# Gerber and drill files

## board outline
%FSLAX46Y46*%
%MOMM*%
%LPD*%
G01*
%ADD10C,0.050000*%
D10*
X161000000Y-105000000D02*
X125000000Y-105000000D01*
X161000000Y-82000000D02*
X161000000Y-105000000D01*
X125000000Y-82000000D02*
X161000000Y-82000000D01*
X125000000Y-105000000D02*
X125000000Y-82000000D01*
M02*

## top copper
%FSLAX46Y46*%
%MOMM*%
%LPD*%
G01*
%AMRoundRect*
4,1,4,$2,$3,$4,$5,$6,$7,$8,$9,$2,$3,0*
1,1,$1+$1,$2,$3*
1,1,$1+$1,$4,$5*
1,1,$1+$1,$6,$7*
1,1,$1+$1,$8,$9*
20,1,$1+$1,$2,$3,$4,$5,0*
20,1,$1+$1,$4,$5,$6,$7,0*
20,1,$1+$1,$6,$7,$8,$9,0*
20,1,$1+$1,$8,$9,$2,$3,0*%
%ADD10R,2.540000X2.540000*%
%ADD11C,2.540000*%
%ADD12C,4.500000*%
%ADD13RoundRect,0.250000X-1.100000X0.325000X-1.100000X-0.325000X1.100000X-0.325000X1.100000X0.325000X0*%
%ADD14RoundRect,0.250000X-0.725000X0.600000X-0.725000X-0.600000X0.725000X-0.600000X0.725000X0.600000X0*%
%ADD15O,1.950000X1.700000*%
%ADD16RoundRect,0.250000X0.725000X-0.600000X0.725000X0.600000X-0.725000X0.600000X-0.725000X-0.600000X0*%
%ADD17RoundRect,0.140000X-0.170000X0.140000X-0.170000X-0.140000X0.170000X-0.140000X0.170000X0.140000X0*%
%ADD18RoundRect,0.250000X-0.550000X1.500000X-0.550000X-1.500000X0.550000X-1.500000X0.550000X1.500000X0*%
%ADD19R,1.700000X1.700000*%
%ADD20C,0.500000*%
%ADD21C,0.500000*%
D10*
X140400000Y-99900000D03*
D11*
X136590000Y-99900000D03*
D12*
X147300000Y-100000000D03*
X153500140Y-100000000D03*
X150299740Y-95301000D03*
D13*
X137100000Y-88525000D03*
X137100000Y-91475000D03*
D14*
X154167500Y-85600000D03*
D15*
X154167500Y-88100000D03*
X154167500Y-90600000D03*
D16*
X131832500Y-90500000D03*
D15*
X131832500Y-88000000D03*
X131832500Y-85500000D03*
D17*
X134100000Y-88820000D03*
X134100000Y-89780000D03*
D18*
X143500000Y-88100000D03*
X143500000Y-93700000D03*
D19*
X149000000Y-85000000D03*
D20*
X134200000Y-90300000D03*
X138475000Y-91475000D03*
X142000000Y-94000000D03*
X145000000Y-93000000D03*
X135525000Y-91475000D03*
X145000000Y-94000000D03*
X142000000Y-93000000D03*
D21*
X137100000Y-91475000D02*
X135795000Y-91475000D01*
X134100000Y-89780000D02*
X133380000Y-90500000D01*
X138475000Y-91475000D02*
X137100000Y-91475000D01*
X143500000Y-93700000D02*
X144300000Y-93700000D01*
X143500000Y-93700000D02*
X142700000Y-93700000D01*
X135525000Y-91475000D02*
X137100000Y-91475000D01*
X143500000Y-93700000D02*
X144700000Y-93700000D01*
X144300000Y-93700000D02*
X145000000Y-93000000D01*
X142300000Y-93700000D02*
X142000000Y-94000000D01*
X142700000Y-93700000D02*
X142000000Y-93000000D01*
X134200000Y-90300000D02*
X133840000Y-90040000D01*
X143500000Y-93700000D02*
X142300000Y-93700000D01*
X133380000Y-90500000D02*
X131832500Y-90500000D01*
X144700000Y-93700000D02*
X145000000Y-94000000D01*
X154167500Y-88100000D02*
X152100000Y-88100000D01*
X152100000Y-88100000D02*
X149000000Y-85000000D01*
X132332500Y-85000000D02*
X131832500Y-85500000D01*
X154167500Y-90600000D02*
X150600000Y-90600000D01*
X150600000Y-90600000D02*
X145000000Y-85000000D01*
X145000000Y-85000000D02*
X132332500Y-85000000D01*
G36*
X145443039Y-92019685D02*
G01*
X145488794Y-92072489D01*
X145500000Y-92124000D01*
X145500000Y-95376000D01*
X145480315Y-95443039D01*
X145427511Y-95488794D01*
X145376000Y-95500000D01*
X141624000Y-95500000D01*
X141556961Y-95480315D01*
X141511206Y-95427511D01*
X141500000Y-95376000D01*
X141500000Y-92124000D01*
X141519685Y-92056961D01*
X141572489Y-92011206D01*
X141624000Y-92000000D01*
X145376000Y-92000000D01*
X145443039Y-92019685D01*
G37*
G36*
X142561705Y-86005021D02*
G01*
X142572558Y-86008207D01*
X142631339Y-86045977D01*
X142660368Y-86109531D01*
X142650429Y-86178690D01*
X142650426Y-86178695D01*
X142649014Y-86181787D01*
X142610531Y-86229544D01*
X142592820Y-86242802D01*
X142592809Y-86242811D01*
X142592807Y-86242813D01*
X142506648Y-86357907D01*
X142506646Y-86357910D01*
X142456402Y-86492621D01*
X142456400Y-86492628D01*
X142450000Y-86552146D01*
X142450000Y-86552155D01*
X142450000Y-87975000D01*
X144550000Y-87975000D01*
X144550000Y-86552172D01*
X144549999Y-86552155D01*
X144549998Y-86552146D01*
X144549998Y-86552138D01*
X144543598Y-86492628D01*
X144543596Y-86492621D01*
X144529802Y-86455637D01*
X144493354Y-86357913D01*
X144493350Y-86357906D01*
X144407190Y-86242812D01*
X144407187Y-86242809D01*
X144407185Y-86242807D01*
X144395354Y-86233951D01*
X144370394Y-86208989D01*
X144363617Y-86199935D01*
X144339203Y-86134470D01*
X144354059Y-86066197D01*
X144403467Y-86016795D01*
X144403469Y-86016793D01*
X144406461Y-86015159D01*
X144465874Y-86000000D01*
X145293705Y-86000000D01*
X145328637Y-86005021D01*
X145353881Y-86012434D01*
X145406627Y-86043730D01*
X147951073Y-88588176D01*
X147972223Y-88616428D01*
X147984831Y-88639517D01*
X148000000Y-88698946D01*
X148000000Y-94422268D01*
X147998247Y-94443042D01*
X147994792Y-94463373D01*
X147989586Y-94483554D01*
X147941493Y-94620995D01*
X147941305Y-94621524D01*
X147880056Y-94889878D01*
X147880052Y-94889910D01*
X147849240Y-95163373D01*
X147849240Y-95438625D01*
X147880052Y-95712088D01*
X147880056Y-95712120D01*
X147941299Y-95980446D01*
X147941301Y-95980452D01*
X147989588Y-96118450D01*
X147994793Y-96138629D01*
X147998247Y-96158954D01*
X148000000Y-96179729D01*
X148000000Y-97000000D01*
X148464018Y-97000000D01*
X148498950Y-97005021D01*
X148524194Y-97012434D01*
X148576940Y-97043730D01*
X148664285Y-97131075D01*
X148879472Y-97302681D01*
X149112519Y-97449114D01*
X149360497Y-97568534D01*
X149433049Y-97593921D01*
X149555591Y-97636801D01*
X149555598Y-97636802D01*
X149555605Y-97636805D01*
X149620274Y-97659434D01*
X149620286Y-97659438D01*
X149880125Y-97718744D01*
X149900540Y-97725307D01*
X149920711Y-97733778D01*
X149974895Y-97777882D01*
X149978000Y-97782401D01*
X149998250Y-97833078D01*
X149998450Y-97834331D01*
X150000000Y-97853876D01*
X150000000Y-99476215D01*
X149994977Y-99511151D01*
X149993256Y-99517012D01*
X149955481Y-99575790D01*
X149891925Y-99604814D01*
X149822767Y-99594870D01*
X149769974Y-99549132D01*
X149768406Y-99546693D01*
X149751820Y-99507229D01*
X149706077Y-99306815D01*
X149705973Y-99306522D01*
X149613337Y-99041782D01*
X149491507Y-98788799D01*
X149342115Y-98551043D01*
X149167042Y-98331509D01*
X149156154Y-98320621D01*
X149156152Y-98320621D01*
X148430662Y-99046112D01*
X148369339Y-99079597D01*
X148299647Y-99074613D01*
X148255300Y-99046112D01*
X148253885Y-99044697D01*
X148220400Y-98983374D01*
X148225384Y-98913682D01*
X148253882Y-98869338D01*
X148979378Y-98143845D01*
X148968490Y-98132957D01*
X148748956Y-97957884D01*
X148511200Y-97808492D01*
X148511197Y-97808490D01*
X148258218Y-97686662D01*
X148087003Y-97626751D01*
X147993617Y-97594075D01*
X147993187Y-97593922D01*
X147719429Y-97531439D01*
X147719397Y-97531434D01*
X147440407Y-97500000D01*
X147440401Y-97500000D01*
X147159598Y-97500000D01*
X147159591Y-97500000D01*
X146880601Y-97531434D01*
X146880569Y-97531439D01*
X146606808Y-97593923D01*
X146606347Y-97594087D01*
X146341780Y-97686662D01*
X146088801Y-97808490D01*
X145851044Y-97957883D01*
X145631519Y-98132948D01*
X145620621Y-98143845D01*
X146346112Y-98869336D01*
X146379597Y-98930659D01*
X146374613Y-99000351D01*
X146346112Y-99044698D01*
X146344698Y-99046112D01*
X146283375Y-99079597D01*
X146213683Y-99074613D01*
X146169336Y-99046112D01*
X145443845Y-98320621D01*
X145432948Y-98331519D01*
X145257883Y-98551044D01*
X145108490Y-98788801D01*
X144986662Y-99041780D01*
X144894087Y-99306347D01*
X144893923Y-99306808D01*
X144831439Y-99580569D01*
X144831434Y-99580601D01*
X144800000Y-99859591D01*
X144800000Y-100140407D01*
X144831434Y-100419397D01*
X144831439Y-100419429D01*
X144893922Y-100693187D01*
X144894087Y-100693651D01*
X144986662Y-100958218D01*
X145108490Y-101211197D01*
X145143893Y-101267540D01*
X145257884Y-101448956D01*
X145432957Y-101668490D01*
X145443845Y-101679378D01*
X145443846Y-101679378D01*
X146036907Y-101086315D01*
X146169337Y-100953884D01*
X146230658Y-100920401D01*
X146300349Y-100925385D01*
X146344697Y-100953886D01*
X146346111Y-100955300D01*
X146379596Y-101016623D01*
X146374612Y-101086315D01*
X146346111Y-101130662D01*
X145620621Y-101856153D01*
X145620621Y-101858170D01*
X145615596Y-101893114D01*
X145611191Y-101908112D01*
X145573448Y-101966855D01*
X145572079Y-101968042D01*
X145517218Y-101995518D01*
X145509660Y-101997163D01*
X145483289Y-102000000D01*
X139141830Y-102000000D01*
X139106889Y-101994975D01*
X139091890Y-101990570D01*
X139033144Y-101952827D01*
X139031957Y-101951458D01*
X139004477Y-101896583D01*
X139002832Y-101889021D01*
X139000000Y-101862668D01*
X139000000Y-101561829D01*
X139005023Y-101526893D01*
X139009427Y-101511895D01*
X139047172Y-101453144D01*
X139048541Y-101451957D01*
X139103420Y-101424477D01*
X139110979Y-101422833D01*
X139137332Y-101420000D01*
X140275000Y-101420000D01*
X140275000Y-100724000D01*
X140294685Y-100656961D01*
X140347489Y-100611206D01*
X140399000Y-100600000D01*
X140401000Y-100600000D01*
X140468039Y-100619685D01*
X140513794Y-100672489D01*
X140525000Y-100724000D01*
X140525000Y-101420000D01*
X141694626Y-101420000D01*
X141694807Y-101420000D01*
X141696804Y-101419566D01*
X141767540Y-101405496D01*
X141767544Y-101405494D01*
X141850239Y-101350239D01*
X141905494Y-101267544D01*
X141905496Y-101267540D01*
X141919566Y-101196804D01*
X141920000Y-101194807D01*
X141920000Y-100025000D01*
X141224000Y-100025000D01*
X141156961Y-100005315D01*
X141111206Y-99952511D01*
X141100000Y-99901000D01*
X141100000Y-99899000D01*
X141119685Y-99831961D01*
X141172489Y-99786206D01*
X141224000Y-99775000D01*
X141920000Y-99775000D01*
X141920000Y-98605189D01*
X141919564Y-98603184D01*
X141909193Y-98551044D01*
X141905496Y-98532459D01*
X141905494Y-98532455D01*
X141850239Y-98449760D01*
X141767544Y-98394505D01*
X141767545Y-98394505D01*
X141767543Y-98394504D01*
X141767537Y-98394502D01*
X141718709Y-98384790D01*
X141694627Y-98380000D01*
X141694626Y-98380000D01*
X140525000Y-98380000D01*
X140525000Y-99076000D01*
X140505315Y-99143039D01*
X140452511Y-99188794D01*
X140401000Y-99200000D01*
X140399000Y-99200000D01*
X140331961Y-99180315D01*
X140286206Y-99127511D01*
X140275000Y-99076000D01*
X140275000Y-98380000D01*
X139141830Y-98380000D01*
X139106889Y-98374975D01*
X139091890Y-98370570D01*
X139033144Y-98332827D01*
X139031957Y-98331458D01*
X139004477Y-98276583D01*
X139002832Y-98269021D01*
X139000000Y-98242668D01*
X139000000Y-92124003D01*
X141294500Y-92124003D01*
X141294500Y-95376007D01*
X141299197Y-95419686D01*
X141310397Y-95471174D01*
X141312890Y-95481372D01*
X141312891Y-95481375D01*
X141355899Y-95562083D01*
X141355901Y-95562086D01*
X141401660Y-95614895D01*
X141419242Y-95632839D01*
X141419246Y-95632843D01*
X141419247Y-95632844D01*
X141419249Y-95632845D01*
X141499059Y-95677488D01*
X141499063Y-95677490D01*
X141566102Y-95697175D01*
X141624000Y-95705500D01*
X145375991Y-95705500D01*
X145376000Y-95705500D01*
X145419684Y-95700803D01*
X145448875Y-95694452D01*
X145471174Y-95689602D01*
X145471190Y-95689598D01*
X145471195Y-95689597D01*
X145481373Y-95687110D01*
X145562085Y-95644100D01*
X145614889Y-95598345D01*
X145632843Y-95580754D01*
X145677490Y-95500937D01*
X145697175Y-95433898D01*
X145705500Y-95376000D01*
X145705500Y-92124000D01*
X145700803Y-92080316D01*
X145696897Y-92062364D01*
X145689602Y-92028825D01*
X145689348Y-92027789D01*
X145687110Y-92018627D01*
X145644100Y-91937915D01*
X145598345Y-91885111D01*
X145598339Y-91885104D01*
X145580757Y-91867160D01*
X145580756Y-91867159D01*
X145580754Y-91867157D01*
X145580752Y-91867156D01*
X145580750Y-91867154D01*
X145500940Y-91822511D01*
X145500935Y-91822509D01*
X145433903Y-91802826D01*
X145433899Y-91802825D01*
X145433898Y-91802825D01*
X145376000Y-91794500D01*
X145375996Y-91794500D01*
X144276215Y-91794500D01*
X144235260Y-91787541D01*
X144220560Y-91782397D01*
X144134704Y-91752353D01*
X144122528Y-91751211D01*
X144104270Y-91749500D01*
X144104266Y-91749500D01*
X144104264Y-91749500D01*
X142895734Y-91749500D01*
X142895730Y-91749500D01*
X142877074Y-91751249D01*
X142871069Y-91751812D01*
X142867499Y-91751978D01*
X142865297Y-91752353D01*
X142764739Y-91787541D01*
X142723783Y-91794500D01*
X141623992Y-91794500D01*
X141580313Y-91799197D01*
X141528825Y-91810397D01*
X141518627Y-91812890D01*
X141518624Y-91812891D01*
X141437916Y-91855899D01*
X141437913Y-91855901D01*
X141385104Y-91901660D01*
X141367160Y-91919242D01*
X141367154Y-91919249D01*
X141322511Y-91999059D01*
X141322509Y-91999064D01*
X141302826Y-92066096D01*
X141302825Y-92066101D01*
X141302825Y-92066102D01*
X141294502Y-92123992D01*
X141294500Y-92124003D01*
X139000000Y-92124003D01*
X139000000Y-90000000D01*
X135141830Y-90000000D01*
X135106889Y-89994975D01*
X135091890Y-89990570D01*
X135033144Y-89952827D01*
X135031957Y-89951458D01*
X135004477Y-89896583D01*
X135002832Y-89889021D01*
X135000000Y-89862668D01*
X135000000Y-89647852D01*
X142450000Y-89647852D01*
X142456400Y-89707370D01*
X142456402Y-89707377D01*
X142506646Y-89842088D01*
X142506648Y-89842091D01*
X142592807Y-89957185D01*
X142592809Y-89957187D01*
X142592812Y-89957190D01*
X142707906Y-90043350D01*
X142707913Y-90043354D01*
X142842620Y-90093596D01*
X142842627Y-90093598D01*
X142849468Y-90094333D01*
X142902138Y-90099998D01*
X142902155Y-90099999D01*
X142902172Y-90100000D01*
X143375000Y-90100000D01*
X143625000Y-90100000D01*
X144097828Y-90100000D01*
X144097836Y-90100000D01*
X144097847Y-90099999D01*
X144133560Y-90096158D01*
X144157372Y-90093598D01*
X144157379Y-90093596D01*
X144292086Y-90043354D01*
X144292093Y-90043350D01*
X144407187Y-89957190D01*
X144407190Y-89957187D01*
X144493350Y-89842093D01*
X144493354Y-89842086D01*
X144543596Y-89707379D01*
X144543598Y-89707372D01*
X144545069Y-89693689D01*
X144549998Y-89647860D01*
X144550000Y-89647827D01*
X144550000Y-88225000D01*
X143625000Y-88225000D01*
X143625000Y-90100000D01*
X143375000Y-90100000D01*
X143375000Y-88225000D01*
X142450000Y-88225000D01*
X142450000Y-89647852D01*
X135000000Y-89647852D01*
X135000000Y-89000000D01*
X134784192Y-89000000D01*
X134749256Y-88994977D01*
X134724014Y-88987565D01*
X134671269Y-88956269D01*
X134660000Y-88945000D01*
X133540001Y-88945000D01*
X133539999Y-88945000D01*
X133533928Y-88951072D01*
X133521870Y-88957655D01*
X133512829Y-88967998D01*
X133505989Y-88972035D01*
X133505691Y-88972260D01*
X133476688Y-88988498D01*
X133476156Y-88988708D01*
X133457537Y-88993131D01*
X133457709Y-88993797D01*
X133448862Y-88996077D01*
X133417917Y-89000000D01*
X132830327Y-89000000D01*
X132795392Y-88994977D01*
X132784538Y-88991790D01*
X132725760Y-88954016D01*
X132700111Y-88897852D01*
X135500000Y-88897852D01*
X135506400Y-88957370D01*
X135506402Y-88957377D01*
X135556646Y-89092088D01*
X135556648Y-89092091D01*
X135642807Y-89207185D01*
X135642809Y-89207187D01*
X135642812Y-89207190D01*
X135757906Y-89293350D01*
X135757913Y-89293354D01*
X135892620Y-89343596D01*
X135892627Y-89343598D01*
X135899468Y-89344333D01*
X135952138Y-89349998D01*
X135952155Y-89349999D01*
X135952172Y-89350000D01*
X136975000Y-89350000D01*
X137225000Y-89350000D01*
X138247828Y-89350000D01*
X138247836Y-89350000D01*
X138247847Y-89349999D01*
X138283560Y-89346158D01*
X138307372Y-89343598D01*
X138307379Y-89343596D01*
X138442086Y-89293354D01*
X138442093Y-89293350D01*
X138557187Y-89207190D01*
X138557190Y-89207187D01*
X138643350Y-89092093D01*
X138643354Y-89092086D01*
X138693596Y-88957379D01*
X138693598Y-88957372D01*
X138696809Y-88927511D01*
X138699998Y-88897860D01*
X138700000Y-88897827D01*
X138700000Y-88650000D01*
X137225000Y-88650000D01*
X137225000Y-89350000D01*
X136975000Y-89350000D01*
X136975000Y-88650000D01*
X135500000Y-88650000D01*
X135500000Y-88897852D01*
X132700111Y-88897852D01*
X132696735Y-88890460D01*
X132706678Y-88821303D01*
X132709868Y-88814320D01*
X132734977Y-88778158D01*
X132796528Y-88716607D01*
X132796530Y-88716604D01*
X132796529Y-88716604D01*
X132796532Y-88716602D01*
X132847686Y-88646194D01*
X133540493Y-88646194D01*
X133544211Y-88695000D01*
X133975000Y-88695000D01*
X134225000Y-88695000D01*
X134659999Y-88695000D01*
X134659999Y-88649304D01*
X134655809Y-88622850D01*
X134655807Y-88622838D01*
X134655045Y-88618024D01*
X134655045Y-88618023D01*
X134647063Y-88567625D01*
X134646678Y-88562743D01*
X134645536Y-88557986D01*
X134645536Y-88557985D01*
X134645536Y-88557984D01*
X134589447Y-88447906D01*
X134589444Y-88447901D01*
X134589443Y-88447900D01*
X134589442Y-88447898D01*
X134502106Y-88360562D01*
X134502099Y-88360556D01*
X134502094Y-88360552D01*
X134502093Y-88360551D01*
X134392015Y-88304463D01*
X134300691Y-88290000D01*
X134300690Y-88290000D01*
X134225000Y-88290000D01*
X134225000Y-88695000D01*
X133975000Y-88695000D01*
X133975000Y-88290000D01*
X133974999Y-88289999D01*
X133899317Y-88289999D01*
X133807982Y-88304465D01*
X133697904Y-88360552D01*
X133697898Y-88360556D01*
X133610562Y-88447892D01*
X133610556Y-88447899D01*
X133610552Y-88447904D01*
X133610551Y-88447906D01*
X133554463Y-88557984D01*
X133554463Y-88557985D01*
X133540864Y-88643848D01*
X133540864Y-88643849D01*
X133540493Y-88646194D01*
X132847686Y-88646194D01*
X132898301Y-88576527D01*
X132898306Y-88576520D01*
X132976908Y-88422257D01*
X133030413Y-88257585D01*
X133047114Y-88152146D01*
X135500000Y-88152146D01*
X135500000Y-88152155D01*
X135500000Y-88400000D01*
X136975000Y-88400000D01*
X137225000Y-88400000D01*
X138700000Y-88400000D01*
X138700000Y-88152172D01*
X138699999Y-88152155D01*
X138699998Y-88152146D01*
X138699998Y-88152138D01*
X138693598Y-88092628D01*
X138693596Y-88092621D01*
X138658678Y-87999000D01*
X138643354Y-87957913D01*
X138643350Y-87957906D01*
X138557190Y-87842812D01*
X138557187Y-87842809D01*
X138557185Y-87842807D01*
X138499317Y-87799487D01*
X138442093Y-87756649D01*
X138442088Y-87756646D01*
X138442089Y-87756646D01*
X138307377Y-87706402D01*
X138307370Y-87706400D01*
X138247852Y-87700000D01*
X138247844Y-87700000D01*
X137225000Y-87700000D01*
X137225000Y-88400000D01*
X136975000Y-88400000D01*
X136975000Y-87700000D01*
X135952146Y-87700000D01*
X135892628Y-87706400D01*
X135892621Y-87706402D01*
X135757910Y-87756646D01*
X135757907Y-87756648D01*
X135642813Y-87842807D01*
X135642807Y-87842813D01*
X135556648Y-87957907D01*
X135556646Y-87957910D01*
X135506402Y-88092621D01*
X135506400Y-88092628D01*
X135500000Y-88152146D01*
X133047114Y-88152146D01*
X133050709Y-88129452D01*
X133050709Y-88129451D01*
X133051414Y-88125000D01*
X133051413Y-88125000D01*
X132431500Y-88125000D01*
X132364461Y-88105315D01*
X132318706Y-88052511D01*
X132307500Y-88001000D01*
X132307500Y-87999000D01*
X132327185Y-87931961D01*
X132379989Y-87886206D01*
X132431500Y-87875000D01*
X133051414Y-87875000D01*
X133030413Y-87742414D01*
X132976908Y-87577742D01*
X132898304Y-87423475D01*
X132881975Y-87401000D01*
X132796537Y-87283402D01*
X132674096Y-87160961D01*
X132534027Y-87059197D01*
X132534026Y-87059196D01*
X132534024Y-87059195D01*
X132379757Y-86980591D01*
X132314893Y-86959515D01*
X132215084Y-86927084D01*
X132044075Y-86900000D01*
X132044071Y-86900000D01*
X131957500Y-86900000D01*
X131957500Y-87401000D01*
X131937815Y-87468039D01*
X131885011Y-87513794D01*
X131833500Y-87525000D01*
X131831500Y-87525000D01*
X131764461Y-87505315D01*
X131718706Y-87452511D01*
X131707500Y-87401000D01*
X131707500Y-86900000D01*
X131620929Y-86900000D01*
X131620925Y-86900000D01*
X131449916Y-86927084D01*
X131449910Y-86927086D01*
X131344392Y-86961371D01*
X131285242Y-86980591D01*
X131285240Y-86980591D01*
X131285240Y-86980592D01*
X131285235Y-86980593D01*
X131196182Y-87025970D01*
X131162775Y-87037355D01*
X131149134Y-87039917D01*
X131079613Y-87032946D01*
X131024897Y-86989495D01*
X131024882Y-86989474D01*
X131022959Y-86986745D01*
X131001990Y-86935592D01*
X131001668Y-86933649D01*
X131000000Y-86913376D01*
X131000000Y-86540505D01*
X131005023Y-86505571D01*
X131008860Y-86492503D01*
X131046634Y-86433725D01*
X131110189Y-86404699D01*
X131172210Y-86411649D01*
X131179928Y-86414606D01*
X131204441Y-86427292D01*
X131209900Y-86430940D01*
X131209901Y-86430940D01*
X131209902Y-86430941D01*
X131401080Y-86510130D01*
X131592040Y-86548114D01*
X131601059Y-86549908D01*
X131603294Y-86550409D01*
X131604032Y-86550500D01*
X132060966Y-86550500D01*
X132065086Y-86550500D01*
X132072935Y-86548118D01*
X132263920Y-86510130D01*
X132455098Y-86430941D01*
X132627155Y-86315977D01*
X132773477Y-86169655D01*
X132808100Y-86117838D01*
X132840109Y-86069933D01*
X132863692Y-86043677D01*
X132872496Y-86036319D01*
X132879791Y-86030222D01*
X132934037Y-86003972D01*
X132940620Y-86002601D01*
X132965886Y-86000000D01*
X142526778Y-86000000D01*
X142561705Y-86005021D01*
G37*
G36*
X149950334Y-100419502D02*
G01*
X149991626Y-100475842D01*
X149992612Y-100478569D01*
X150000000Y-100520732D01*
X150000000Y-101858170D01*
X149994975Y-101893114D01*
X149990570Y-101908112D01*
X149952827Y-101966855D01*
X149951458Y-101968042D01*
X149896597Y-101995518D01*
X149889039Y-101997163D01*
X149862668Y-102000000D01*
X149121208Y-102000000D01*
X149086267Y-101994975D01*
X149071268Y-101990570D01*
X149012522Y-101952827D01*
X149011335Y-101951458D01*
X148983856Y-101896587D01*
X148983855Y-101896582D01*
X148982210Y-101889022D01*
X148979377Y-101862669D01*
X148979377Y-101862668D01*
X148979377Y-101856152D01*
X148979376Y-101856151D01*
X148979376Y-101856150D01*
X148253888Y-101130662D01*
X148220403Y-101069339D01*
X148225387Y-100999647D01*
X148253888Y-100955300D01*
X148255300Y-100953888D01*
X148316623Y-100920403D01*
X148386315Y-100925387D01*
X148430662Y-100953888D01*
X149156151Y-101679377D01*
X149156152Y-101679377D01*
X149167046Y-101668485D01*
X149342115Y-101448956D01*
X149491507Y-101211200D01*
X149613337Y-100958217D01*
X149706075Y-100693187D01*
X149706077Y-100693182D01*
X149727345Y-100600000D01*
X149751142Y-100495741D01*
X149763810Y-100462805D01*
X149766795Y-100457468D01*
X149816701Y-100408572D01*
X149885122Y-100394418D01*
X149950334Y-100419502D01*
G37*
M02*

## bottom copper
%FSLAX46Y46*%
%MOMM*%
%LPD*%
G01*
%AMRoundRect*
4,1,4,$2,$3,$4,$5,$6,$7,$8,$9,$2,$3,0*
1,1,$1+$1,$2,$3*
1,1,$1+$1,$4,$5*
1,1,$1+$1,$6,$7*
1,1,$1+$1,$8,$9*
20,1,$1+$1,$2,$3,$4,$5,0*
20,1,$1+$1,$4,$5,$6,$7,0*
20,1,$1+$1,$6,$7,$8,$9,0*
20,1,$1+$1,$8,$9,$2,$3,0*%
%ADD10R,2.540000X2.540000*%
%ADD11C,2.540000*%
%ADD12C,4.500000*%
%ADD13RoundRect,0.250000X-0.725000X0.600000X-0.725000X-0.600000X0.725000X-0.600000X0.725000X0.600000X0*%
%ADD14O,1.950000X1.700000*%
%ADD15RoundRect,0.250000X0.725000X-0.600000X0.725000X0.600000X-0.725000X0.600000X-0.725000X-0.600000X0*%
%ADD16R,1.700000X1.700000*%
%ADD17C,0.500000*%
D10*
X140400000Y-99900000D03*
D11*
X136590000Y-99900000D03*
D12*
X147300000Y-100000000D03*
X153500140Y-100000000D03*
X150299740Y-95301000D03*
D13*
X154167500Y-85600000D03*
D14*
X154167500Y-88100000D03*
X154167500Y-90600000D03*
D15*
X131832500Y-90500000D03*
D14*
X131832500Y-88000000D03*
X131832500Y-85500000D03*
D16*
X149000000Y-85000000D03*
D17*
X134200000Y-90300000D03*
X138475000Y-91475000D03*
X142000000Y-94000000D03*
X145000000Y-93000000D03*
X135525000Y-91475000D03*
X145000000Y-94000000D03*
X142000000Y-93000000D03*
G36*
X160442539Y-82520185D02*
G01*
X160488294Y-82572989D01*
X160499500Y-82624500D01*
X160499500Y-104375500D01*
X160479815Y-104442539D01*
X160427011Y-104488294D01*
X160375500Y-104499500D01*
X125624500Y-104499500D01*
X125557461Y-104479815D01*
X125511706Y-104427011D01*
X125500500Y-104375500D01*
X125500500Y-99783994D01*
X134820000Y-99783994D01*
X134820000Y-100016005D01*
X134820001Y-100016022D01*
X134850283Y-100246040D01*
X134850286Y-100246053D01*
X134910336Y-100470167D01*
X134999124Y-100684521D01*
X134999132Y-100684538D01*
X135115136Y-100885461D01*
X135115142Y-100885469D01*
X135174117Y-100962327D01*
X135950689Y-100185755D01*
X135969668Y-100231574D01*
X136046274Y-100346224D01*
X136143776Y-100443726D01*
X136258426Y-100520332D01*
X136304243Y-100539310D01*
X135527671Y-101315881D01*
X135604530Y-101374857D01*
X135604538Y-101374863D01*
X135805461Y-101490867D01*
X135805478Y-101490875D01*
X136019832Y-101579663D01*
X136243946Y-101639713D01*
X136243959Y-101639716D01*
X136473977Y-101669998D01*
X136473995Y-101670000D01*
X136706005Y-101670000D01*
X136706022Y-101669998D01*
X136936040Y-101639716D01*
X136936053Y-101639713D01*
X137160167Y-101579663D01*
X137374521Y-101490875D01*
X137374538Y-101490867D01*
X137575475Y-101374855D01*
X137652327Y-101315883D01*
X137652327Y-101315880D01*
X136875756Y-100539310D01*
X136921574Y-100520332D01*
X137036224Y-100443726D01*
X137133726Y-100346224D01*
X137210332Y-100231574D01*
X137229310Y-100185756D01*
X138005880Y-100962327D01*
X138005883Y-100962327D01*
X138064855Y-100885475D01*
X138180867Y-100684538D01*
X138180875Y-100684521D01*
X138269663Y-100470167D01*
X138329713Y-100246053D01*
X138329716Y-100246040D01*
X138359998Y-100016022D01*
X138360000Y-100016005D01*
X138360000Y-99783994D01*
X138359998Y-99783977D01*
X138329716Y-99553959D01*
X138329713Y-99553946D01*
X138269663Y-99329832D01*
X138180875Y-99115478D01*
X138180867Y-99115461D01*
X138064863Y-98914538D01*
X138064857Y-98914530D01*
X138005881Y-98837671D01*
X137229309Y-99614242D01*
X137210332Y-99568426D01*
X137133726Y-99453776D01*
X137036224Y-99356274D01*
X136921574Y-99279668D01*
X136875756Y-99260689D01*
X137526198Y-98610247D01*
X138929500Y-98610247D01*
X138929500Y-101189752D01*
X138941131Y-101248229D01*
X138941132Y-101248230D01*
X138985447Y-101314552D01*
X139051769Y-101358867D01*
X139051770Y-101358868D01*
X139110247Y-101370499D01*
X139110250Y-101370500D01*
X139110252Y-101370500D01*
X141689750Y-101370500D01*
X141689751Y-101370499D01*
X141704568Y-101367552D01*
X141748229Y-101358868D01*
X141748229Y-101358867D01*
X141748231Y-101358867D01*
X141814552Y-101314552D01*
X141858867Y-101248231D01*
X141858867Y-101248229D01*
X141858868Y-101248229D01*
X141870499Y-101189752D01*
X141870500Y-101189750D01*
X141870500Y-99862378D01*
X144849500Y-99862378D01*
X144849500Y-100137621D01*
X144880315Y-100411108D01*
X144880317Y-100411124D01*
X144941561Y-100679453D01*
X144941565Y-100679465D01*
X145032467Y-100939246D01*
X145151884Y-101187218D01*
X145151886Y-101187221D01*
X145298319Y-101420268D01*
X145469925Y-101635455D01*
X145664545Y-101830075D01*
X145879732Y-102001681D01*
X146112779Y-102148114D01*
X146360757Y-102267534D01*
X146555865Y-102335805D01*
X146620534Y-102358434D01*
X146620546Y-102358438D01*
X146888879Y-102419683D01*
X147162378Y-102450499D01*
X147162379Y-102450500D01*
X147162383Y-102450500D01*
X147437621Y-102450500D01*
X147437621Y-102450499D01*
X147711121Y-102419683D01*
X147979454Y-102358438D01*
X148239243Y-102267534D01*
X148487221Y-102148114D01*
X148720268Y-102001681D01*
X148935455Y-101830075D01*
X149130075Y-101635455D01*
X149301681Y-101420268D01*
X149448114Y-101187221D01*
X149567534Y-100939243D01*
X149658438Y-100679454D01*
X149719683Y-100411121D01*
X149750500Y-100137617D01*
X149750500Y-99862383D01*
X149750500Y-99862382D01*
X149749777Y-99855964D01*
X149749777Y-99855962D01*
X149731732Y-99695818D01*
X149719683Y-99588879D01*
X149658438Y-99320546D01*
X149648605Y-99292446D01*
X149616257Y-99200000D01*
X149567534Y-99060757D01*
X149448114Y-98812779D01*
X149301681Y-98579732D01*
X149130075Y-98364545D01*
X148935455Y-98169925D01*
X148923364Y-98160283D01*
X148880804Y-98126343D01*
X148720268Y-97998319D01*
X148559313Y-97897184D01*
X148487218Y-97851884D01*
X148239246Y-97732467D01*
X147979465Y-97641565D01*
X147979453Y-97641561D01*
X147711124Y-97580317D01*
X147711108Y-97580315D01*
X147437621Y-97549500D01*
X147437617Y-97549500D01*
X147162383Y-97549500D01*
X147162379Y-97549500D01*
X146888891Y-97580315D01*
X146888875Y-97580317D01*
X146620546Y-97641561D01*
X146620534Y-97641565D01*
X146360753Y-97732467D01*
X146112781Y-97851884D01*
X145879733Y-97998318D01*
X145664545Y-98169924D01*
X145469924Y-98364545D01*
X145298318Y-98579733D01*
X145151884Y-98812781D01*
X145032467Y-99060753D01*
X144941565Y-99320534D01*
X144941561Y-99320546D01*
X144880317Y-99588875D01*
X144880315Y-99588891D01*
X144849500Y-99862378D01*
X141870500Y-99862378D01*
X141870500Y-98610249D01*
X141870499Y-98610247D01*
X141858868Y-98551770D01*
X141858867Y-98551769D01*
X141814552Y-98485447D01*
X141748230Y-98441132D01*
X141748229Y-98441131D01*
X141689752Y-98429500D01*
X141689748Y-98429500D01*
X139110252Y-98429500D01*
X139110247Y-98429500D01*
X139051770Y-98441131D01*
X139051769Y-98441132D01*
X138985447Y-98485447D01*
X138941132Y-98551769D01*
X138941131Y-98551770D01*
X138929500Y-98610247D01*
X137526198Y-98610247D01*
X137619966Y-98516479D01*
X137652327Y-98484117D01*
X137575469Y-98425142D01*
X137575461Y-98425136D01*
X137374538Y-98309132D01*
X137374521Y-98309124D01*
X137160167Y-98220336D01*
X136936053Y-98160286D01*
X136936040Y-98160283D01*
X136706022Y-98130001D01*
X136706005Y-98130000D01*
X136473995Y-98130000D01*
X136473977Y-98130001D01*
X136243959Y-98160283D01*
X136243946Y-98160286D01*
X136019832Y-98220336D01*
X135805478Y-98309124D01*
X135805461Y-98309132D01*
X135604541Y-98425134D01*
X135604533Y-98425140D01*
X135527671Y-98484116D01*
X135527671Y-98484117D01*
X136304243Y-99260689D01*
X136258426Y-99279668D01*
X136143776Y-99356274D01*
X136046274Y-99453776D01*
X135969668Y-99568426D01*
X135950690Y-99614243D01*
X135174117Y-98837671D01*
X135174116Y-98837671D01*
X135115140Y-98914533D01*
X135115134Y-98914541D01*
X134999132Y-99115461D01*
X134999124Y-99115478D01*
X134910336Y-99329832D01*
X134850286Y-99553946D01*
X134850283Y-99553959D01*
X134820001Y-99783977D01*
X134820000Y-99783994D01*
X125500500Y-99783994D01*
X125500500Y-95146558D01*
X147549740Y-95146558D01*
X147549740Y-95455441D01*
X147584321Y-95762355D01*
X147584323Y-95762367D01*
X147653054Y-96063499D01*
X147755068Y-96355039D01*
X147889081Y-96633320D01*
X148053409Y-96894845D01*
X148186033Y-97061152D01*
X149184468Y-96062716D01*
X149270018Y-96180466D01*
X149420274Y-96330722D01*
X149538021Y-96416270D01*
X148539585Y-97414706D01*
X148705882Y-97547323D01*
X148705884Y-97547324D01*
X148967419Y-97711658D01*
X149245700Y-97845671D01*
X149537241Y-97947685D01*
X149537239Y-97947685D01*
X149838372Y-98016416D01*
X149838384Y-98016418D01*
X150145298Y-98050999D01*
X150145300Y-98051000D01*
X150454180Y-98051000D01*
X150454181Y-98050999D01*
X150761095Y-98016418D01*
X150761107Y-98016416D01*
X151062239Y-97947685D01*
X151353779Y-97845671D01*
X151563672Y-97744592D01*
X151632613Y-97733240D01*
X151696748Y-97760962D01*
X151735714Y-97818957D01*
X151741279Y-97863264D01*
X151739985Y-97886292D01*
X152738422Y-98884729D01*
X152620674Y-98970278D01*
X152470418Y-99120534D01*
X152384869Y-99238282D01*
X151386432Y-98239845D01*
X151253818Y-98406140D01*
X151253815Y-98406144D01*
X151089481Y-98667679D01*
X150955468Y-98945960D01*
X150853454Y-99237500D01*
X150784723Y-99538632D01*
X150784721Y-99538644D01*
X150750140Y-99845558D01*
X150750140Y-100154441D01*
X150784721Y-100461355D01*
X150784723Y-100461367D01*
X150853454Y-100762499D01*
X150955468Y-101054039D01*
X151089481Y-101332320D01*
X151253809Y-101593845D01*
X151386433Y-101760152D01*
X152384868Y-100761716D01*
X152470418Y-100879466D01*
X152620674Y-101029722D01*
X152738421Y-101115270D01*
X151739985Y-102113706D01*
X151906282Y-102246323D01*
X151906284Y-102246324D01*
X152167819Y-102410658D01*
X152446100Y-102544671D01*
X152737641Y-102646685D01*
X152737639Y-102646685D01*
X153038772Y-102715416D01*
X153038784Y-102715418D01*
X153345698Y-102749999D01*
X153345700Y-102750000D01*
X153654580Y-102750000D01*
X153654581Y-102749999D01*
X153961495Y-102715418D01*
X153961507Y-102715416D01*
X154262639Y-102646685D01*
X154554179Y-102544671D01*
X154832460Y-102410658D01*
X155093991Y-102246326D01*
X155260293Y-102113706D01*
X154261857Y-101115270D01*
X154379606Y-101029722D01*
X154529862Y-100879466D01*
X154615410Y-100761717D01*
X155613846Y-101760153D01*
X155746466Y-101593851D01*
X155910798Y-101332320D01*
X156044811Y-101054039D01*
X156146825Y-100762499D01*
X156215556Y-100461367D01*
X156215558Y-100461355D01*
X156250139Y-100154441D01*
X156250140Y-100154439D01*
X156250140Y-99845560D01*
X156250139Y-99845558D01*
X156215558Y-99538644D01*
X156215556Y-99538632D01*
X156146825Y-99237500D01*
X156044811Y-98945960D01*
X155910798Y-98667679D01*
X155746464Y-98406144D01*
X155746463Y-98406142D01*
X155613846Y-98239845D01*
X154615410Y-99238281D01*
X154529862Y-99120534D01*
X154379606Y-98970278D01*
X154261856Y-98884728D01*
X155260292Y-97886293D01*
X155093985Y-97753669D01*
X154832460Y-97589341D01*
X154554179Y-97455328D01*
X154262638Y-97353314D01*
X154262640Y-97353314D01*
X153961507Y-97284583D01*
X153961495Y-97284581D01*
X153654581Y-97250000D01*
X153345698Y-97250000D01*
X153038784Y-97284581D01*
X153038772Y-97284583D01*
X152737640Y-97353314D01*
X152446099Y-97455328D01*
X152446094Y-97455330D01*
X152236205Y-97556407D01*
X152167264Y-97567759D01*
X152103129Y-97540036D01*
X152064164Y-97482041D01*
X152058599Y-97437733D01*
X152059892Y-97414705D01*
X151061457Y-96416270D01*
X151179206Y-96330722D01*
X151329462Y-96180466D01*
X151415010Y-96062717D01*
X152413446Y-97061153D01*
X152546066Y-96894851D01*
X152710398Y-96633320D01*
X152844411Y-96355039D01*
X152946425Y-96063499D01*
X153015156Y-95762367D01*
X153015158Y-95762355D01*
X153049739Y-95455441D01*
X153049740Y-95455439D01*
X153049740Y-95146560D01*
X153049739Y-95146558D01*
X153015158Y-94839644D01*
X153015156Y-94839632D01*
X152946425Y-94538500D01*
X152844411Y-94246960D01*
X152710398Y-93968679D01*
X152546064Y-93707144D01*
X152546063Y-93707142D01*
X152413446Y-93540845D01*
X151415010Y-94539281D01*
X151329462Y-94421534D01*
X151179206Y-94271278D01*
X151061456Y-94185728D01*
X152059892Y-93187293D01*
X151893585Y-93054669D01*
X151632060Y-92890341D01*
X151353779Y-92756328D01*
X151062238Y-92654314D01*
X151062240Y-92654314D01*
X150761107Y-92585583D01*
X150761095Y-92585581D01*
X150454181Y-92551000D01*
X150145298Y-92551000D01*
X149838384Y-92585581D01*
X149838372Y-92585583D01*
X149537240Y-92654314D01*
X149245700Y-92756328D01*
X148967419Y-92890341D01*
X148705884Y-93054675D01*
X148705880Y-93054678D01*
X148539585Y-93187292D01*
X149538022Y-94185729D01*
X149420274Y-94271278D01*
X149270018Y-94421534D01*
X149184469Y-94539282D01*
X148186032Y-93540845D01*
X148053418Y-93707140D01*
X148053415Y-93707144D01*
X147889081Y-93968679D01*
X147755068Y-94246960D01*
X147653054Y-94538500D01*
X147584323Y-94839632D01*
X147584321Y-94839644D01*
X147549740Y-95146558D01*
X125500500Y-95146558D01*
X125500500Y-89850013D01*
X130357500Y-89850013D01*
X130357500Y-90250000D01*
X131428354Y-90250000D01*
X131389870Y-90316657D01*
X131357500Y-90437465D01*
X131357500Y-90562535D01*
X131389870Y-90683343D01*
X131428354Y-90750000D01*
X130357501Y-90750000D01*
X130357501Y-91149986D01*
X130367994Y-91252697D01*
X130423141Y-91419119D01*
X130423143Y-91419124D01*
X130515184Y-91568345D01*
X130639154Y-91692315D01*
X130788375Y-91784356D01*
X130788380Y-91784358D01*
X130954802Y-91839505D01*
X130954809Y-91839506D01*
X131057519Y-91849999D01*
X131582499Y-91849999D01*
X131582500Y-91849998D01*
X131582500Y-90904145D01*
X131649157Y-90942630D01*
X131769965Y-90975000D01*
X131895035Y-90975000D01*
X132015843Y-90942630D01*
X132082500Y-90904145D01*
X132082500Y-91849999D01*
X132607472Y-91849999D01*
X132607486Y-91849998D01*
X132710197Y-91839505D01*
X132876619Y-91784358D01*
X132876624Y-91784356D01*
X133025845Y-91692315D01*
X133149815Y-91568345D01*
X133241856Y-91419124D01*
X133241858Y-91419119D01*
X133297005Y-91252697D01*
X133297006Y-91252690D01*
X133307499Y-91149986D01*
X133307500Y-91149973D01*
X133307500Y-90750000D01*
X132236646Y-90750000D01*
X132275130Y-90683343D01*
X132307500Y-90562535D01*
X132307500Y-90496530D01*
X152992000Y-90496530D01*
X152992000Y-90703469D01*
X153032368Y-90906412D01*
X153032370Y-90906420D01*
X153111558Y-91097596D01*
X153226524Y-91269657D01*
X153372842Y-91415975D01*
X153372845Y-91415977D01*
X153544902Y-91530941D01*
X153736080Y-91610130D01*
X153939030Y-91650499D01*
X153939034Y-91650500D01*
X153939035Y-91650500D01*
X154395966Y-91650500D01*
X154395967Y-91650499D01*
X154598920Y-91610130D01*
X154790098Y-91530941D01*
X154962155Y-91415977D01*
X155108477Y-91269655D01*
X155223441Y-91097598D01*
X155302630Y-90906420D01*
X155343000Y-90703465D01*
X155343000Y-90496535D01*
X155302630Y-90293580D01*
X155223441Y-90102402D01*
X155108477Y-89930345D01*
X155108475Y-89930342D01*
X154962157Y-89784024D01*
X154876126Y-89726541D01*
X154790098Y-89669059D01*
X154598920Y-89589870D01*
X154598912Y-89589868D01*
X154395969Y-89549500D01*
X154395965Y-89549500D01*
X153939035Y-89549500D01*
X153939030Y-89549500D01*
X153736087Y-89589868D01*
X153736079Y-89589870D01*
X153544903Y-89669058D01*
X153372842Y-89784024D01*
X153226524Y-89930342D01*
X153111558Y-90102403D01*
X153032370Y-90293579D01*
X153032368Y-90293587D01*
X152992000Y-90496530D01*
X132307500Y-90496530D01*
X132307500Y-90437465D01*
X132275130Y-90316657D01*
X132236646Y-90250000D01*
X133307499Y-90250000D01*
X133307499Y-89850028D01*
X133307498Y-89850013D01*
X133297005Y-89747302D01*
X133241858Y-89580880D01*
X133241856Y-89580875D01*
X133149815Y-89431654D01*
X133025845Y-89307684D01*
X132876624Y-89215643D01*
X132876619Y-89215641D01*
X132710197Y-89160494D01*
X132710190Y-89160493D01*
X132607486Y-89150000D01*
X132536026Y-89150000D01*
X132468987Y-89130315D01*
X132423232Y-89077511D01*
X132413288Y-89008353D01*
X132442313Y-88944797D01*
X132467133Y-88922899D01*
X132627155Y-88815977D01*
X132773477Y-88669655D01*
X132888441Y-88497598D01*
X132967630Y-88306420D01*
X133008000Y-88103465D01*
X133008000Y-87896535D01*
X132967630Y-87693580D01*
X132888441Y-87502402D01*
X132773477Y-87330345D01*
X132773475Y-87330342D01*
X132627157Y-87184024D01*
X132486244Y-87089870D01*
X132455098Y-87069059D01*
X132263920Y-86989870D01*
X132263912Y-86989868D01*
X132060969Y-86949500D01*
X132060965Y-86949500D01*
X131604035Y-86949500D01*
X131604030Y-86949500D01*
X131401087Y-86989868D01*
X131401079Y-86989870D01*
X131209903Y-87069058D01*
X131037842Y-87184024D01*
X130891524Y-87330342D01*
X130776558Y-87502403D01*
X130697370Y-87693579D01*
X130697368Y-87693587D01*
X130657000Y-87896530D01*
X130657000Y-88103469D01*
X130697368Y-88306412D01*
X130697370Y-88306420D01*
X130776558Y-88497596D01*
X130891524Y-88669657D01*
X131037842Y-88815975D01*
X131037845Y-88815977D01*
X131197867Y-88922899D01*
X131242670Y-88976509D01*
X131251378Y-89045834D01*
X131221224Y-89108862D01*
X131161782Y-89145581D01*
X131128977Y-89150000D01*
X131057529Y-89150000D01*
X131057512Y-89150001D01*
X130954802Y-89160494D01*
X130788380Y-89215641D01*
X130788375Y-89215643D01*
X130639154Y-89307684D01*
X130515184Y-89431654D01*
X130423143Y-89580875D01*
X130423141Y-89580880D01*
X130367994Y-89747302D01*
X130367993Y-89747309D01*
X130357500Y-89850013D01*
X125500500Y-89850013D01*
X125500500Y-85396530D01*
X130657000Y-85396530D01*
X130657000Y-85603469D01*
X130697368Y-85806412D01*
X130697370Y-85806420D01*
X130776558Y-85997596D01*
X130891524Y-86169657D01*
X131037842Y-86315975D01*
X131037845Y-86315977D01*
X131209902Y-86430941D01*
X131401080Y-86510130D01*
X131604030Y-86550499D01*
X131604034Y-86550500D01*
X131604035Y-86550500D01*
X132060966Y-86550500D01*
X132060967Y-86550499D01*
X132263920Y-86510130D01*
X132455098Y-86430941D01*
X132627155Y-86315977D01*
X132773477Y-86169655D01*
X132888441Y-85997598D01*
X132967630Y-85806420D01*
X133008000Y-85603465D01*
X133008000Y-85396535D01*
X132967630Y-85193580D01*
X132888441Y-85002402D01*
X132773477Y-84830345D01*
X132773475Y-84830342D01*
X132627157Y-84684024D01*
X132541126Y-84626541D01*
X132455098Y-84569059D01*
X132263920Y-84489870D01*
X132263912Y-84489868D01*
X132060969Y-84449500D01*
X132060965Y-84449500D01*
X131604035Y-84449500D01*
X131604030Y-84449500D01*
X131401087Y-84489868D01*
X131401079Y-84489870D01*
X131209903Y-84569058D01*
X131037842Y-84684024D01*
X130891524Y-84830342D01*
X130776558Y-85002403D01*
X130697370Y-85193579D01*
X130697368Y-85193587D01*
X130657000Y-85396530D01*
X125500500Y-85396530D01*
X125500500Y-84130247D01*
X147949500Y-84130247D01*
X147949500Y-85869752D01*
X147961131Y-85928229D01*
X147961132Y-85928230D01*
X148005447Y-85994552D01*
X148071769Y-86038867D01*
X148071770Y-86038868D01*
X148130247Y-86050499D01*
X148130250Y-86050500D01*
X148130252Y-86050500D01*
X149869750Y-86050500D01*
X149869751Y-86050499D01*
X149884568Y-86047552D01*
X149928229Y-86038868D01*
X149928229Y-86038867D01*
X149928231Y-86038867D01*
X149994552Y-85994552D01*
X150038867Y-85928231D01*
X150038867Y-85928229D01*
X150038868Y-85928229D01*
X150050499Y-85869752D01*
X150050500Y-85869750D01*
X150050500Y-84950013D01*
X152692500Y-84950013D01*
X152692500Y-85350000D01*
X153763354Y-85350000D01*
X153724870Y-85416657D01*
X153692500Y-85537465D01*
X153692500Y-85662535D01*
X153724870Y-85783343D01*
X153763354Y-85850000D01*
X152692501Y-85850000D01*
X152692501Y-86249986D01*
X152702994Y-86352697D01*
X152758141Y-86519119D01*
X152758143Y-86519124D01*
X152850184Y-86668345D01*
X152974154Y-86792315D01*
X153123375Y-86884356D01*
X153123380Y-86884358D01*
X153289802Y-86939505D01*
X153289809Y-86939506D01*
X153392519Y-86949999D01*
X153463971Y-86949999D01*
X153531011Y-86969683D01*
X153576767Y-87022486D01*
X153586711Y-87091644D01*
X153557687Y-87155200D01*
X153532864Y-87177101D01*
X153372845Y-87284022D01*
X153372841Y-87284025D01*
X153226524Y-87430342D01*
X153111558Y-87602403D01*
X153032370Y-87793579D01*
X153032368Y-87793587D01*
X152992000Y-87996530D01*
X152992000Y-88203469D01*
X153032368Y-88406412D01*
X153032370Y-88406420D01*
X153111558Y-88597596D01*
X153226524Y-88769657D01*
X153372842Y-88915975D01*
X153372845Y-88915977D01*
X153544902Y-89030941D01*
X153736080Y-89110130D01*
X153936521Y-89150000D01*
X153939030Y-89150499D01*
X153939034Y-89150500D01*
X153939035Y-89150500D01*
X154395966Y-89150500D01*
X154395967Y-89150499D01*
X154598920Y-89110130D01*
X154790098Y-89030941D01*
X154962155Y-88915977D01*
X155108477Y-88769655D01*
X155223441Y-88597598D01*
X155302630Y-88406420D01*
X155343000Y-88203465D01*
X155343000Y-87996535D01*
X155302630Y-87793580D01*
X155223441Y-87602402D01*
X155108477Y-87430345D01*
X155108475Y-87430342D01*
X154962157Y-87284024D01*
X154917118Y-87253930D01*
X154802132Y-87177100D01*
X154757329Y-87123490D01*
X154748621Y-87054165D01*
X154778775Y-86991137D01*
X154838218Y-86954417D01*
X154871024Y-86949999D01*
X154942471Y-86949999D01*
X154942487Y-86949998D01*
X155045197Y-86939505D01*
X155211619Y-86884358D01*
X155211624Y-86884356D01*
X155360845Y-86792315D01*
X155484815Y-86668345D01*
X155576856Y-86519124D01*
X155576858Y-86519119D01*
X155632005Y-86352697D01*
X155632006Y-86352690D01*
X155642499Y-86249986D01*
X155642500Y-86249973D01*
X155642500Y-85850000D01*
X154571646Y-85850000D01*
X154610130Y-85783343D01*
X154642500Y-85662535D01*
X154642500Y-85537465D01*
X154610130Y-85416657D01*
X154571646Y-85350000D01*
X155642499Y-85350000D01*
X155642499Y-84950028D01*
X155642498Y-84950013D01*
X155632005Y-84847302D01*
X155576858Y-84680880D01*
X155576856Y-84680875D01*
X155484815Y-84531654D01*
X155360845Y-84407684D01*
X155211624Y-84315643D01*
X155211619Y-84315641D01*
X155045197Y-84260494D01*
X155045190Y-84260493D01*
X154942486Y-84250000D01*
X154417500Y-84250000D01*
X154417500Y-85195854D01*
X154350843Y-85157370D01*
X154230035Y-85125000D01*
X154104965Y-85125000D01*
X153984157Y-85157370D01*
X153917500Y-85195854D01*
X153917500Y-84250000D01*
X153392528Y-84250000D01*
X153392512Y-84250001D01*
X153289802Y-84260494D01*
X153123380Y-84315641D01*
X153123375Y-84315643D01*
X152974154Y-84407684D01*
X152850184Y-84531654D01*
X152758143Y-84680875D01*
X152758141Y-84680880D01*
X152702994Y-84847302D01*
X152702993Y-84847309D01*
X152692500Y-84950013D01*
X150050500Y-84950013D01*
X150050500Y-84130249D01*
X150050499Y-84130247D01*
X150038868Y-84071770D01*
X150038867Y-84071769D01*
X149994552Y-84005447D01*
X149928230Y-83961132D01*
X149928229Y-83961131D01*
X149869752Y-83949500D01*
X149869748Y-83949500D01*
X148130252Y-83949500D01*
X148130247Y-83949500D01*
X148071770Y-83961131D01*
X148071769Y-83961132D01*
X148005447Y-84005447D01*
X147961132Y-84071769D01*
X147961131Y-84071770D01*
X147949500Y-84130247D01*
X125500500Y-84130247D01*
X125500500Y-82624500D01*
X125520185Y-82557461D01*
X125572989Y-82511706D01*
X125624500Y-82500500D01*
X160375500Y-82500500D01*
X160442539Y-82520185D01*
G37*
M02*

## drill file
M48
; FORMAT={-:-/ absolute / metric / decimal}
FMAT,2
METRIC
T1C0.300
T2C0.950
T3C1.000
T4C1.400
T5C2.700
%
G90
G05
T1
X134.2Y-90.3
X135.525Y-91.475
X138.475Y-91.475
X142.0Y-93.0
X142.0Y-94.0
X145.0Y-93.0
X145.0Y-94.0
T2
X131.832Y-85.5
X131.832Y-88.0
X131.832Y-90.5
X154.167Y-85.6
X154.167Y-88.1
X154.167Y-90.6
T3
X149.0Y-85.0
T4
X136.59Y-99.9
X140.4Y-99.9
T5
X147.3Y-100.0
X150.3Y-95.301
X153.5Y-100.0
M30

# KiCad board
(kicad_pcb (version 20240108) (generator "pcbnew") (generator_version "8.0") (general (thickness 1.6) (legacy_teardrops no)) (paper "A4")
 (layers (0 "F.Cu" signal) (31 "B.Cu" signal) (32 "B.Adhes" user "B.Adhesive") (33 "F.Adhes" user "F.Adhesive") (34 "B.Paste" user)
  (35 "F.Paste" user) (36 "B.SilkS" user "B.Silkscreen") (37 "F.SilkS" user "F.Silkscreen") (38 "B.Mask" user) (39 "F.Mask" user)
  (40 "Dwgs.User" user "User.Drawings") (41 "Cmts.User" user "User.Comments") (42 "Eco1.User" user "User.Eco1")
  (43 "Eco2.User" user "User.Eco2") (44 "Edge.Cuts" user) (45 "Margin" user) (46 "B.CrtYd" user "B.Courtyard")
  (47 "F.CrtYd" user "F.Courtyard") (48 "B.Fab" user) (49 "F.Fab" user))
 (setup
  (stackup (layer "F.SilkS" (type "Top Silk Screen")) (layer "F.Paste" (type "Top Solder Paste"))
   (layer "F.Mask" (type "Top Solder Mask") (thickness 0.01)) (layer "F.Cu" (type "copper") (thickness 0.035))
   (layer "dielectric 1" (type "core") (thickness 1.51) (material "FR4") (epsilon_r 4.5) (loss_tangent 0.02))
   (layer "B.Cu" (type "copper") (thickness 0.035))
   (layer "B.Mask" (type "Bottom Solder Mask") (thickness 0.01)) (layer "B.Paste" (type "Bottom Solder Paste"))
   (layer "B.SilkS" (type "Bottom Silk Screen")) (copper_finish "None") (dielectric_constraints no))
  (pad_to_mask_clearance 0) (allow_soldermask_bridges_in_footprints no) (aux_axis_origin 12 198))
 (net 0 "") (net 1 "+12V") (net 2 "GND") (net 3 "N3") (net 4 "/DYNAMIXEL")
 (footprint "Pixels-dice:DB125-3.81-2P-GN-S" (layer "F.Cu") (at 140.4 99.9 180)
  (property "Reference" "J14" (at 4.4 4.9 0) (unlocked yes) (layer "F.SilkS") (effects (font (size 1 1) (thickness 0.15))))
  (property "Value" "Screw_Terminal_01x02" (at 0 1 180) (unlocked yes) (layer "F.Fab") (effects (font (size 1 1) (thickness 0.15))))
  (pad "1" thru_hole rect (at 0 0 180) (size 2.54 2.54) (drill 1.4) (layers "*.Cu" "*.Mask") (remove_unused_layers no) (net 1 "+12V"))
  (pad "2" thru_hole circle (at 3.81 0 180) (size 2.54 2.54) (drill 1.4) (layers "*.Cu" "*.Mask") (remove_unused_layers no) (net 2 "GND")))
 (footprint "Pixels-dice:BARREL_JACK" (layer "F.Cu") (at 153.50014 100 180)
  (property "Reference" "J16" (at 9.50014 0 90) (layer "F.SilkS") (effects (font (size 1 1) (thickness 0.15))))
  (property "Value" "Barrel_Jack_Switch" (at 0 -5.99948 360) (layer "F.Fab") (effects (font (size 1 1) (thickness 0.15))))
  (pad "1" thru_hole circle (at 6.20014 0 180) (size 4.5 4.5) (drill 2.7) (layers "*.Cu" "*.Mask" "F.SilkS") (remove_unused_layers no)
   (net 1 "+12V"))
  (pad "2" thru_hole circle (at 0 0 180) (size 4.5 4.5) (drill 2.7) (layers "*.Cu" "*.Mask" "F.SilkS") (remove_unused_layers no)
   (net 2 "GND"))
  (pad "3" thru_hole circle (at 3.2004 4.699 180) (size 4.5 4.5) (drill 2.7) (layers "*.Cu" "*.Mask" "F.SilkS") (remove_unused_layers no)
   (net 2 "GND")))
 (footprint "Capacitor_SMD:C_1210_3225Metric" (layer "F.Cu") (at 137.1 90 -90)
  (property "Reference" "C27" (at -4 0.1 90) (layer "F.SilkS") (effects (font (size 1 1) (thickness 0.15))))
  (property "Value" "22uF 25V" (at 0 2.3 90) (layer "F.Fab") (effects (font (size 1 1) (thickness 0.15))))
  (pad "1" smd roundrect (at -1.475 0 270) (size 1.15 2.7) (layers "F.Cu" "F.Paste" "F.Mask") (roundrect_rratio 0.217391) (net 1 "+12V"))
  (pad "2" smd roundrect (at 1.475 0 270) (size 1.15 2.7) (layers "F.Cu" "F.Paste" "F.Mask") (roundrect_rratio 0.217391) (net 2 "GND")))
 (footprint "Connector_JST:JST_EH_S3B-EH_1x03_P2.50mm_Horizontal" (layer "F.Cu") (at 154.1675 85.6 -90)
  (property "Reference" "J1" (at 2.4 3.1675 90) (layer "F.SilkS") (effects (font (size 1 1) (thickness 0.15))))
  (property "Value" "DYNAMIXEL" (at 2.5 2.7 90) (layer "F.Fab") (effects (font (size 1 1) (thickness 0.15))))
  (pad "1" thru_hole roundrect (at 0 0 270) (size 1.7 1.95) (drill 0.95) (layers "*.Cu" "*.Mask") (remove_unused_layers no)
   (roundrect_rratio 0.147059) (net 2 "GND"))
  (pad "2" thru_hole oval (at 2.5 0 270) (size 1.7 1.95) (drill 0.95) (layers "*.Cu" "*.Mask") (remove_unused_layers no) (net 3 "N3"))
  (pad "3" thru_hole oval (at 5 0 270) (size 1.7 1.95) (drill 0.95) (layers "*.Cu" "*.Mask") (remove_unused_layers no) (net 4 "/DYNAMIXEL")))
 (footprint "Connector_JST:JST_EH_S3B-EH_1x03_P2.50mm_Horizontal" (layer "F.Cu") (at 131.8325 90.5 90)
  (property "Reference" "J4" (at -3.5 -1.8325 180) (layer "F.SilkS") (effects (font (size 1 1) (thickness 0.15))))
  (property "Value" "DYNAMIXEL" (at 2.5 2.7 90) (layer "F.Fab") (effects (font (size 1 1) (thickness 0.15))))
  (pad "1" thru_hole roundrect (at 0 0 90) (size 1.7 1.95) (drill 0.95) (layers "*.Cu" "*.Mask") (remove_unused_layers no)
   (roundrect_rratio 0.147059) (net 2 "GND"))
  (pad "2" thru_hole oval (at 2.5 0 90) (size 1.7 1.95) (drill 0.95) (layers "*.Cu" "*.Mask") (remove_unused_layers no) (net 1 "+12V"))
  (pad "3" thru_hole oval (at 5 0 90) (size 1.7 1.95) (drill 0.95) (layers "*.Cu" "*.Mask") (remove_unused_layers no) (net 4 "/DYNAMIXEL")))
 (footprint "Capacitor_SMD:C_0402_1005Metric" (layer "F.Cu") (at 134.1 89.3 -90)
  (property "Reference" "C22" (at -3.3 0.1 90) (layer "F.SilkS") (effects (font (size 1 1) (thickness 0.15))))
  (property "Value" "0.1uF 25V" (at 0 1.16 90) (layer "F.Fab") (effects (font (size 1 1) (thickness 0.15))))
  (pad "1" smd roundrect (at -0.48 0 270) (size 0.56 0.62) (layers "F.Cu" "F.Paste" "F.Mask") (roundrect_rratio 0.25) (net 1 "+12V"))
  (pad "2" smd roundrect (at 0.48 0 270) (size 0.56 0.62) (layers "F.Cu" "F.Paste" "F.Mask") (roundrect_rratio 0.25) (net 2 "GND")))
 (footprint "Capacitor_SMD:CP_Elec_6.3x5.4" (layer "F.Cu") (at 143.5 90.9 -90)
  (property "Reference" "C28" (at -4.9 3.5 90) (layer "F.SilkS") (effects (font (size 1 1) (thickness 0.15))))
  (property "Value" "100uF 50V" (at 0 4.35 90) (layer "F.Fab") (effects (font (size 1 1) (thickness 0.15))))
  (pad "1" smd roundrect (at -2.8 0 270) (size 3.5 1.6) (layers "F.Cu" "F.Paste" "F.Mask") (roundrect_rratio 0.15625) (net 1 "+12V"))
  (pad "2" smd roundrect (at 2.8 0 270) (size 3.5 1.6) (layers "F.Cu" "F.Paste" "F.Mask") (roundrect_rratio 0.15625) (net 2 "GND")))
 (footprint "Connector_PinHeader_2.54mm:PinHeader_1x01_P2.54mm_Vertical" (layer "F.Cu") (at 149 85)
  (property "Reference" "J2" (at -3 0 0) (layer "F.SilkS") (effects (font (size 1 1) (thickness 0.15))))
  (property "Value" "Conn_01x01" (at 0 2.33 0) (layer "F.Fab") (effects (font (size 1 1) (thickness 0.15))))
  (pad "1" thru_hole rect (at 0 0) (size 1.7 1.7) (drill 1) (layers "*.Cu" "*.Mask") (remove_unused_layers no) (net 3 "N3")))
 (gr_line (start 161 105) (end 125 105) (stroke (width 0.05) (type default)) (layer "Edge.Cuts"))
 (gr_line (start 161 82) (end 161 105) (stroke (width 0.05) (type default)) (layer "Edge.Cuts"))
 (gr_line (start 125 82) (end 161 82) (stroke (width 0.05) (type default)) (layer "Edge.Cuts"))
 (gr_line (start 125 105) (end 125 82) (stroke (width 0.05) (type default)) (layer "Edge.Cuts"))
 (segment (start 137.1 91.475) (end 135.795 91.475) (width 0.5) (layer "F.Cu") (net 2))
 (segment (start 134.1 89.78) (end 133.38 90.5) (width 0.5) (layer "F.Cu") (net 2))
 (segment (start 138.475 91.475) (end 137.1 91.475) (width 0.5) (layer "F.Cu") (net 2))
 (segment (start 143.5 93.7) (end 144.3 93.7) (width 0.5) (layer "F.Cu") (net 2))
 (segment (start 143.5 93.7) (end 142.7 93.7) (width 0.5) (layer "F.Cu") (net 2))
 (segment (start 135.525 91.475) (end 137.1 91.475) (width 0.5) (layer "F.Cu") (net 2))
 (segment (start 143.5 93.7) (end 144.7 93.7) (width 0.5) (layer "F.Cu") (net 2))
 (segment (start 144.3 93.7) (end 145 93) (width 0.5) (layer "F.Cu") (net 2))
 (segment (start 142.3 93.7) (end 142 94) (width 0.5) (layer "F.Cu") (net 2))
 (segment (start 142.7 93.7) (end 142 93) (width 0.5) (layer "F.Cu") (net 2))
 (segment (start 134.2 90.3) (end 133.84 90.04) (width 0.5) (layer "F.Cu") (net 2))
 (segment (start 143.5 93.7) (end 142.3 93.7) (width 0.5) (layer "F.Cu") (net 2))
 (segment (start 133.38 90.5) (end 131.8325 90.5) (width 0.5) (layer "F.Cu") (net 2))
 (segment (start 144.7 93.7) (end 145 94) (width 0.5) (layer "F.Cu") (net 2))
 (via (at 134.2 90.3) (size 0.5) (drill 0.3) (layers "F.Cu" "B.Cu") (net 2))
 (via (at 138.475 91.475) (size 0.5) (drill 0.3) (layers "F.Cu" "B.Cu") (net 2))
 (via (at 142 94) (size 0.5) (drill 0.3) (layers "F.Cu" "B.Cu") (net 2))
 (via (at 145 93) (size 0.5) (drill 0.3) (layers "F.Cu" "B.Cu") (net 2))
 (via (at 135.525 91.475) (size 0.5) (drill 0.3) (layers "F.Cu" "B.Cu") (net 2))
 (via (at 145 94) (size 0.5) (drill 0.3) (layers "F.Cu" "B.Cu") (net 2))
 (via (at 142 93) (size 0.5) (drill 0.3) (layers "F.Cu" "B.Cu") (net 2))
 (segment (start 154.1675 88.1) (end 152.1 88.1) (width 0.5) (layer "F.Cu") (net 3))
 (segment (start 152.1 88.1) (end 149 85) (width 0.5) (layer "F.Cu") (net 3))
 (segment (start 132.3325 85) (end 131.8325 85.5) (width 0.5) (layer "F.Cu") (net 4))
 (segment (start 154.1675 90.6) (end 150.6 90.6) (width 0.5) (layer "F.Cu") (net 4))
 (segment (start 150.6 90.6) (end 145 85) (width 0.5) (layer "F.Cu") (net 4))
 (segment (start 145 85) (end 132.3325 85) (width 0.5) (layer "F.Cu") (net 4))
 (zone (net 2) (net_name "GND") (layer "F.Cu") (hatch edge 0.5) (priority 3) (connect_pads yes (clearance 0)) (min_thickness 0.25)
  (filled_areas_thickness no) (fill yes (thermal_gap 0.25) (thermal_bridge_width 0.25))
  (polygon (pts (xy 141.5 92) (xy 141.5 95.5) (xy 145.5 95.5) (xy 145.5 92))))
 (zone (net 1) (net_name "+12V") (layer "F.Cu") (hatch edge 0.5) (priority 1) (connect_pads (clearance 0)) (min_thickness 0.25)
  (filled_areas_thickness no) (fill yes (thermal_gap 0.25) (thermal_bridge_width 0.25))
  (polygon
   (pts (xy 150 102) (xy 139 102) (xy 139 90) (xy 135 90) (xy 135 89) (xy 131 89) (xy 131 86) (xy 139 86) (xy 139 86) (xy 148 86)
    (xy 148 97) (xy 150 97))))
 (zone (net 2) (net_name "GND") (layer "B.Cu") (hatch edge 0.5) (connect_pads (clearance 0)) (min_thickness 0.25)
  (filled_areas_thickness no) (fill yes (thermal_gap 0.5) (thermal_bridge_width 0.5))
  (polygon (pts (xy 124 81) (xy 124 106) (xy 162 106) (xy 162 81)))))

